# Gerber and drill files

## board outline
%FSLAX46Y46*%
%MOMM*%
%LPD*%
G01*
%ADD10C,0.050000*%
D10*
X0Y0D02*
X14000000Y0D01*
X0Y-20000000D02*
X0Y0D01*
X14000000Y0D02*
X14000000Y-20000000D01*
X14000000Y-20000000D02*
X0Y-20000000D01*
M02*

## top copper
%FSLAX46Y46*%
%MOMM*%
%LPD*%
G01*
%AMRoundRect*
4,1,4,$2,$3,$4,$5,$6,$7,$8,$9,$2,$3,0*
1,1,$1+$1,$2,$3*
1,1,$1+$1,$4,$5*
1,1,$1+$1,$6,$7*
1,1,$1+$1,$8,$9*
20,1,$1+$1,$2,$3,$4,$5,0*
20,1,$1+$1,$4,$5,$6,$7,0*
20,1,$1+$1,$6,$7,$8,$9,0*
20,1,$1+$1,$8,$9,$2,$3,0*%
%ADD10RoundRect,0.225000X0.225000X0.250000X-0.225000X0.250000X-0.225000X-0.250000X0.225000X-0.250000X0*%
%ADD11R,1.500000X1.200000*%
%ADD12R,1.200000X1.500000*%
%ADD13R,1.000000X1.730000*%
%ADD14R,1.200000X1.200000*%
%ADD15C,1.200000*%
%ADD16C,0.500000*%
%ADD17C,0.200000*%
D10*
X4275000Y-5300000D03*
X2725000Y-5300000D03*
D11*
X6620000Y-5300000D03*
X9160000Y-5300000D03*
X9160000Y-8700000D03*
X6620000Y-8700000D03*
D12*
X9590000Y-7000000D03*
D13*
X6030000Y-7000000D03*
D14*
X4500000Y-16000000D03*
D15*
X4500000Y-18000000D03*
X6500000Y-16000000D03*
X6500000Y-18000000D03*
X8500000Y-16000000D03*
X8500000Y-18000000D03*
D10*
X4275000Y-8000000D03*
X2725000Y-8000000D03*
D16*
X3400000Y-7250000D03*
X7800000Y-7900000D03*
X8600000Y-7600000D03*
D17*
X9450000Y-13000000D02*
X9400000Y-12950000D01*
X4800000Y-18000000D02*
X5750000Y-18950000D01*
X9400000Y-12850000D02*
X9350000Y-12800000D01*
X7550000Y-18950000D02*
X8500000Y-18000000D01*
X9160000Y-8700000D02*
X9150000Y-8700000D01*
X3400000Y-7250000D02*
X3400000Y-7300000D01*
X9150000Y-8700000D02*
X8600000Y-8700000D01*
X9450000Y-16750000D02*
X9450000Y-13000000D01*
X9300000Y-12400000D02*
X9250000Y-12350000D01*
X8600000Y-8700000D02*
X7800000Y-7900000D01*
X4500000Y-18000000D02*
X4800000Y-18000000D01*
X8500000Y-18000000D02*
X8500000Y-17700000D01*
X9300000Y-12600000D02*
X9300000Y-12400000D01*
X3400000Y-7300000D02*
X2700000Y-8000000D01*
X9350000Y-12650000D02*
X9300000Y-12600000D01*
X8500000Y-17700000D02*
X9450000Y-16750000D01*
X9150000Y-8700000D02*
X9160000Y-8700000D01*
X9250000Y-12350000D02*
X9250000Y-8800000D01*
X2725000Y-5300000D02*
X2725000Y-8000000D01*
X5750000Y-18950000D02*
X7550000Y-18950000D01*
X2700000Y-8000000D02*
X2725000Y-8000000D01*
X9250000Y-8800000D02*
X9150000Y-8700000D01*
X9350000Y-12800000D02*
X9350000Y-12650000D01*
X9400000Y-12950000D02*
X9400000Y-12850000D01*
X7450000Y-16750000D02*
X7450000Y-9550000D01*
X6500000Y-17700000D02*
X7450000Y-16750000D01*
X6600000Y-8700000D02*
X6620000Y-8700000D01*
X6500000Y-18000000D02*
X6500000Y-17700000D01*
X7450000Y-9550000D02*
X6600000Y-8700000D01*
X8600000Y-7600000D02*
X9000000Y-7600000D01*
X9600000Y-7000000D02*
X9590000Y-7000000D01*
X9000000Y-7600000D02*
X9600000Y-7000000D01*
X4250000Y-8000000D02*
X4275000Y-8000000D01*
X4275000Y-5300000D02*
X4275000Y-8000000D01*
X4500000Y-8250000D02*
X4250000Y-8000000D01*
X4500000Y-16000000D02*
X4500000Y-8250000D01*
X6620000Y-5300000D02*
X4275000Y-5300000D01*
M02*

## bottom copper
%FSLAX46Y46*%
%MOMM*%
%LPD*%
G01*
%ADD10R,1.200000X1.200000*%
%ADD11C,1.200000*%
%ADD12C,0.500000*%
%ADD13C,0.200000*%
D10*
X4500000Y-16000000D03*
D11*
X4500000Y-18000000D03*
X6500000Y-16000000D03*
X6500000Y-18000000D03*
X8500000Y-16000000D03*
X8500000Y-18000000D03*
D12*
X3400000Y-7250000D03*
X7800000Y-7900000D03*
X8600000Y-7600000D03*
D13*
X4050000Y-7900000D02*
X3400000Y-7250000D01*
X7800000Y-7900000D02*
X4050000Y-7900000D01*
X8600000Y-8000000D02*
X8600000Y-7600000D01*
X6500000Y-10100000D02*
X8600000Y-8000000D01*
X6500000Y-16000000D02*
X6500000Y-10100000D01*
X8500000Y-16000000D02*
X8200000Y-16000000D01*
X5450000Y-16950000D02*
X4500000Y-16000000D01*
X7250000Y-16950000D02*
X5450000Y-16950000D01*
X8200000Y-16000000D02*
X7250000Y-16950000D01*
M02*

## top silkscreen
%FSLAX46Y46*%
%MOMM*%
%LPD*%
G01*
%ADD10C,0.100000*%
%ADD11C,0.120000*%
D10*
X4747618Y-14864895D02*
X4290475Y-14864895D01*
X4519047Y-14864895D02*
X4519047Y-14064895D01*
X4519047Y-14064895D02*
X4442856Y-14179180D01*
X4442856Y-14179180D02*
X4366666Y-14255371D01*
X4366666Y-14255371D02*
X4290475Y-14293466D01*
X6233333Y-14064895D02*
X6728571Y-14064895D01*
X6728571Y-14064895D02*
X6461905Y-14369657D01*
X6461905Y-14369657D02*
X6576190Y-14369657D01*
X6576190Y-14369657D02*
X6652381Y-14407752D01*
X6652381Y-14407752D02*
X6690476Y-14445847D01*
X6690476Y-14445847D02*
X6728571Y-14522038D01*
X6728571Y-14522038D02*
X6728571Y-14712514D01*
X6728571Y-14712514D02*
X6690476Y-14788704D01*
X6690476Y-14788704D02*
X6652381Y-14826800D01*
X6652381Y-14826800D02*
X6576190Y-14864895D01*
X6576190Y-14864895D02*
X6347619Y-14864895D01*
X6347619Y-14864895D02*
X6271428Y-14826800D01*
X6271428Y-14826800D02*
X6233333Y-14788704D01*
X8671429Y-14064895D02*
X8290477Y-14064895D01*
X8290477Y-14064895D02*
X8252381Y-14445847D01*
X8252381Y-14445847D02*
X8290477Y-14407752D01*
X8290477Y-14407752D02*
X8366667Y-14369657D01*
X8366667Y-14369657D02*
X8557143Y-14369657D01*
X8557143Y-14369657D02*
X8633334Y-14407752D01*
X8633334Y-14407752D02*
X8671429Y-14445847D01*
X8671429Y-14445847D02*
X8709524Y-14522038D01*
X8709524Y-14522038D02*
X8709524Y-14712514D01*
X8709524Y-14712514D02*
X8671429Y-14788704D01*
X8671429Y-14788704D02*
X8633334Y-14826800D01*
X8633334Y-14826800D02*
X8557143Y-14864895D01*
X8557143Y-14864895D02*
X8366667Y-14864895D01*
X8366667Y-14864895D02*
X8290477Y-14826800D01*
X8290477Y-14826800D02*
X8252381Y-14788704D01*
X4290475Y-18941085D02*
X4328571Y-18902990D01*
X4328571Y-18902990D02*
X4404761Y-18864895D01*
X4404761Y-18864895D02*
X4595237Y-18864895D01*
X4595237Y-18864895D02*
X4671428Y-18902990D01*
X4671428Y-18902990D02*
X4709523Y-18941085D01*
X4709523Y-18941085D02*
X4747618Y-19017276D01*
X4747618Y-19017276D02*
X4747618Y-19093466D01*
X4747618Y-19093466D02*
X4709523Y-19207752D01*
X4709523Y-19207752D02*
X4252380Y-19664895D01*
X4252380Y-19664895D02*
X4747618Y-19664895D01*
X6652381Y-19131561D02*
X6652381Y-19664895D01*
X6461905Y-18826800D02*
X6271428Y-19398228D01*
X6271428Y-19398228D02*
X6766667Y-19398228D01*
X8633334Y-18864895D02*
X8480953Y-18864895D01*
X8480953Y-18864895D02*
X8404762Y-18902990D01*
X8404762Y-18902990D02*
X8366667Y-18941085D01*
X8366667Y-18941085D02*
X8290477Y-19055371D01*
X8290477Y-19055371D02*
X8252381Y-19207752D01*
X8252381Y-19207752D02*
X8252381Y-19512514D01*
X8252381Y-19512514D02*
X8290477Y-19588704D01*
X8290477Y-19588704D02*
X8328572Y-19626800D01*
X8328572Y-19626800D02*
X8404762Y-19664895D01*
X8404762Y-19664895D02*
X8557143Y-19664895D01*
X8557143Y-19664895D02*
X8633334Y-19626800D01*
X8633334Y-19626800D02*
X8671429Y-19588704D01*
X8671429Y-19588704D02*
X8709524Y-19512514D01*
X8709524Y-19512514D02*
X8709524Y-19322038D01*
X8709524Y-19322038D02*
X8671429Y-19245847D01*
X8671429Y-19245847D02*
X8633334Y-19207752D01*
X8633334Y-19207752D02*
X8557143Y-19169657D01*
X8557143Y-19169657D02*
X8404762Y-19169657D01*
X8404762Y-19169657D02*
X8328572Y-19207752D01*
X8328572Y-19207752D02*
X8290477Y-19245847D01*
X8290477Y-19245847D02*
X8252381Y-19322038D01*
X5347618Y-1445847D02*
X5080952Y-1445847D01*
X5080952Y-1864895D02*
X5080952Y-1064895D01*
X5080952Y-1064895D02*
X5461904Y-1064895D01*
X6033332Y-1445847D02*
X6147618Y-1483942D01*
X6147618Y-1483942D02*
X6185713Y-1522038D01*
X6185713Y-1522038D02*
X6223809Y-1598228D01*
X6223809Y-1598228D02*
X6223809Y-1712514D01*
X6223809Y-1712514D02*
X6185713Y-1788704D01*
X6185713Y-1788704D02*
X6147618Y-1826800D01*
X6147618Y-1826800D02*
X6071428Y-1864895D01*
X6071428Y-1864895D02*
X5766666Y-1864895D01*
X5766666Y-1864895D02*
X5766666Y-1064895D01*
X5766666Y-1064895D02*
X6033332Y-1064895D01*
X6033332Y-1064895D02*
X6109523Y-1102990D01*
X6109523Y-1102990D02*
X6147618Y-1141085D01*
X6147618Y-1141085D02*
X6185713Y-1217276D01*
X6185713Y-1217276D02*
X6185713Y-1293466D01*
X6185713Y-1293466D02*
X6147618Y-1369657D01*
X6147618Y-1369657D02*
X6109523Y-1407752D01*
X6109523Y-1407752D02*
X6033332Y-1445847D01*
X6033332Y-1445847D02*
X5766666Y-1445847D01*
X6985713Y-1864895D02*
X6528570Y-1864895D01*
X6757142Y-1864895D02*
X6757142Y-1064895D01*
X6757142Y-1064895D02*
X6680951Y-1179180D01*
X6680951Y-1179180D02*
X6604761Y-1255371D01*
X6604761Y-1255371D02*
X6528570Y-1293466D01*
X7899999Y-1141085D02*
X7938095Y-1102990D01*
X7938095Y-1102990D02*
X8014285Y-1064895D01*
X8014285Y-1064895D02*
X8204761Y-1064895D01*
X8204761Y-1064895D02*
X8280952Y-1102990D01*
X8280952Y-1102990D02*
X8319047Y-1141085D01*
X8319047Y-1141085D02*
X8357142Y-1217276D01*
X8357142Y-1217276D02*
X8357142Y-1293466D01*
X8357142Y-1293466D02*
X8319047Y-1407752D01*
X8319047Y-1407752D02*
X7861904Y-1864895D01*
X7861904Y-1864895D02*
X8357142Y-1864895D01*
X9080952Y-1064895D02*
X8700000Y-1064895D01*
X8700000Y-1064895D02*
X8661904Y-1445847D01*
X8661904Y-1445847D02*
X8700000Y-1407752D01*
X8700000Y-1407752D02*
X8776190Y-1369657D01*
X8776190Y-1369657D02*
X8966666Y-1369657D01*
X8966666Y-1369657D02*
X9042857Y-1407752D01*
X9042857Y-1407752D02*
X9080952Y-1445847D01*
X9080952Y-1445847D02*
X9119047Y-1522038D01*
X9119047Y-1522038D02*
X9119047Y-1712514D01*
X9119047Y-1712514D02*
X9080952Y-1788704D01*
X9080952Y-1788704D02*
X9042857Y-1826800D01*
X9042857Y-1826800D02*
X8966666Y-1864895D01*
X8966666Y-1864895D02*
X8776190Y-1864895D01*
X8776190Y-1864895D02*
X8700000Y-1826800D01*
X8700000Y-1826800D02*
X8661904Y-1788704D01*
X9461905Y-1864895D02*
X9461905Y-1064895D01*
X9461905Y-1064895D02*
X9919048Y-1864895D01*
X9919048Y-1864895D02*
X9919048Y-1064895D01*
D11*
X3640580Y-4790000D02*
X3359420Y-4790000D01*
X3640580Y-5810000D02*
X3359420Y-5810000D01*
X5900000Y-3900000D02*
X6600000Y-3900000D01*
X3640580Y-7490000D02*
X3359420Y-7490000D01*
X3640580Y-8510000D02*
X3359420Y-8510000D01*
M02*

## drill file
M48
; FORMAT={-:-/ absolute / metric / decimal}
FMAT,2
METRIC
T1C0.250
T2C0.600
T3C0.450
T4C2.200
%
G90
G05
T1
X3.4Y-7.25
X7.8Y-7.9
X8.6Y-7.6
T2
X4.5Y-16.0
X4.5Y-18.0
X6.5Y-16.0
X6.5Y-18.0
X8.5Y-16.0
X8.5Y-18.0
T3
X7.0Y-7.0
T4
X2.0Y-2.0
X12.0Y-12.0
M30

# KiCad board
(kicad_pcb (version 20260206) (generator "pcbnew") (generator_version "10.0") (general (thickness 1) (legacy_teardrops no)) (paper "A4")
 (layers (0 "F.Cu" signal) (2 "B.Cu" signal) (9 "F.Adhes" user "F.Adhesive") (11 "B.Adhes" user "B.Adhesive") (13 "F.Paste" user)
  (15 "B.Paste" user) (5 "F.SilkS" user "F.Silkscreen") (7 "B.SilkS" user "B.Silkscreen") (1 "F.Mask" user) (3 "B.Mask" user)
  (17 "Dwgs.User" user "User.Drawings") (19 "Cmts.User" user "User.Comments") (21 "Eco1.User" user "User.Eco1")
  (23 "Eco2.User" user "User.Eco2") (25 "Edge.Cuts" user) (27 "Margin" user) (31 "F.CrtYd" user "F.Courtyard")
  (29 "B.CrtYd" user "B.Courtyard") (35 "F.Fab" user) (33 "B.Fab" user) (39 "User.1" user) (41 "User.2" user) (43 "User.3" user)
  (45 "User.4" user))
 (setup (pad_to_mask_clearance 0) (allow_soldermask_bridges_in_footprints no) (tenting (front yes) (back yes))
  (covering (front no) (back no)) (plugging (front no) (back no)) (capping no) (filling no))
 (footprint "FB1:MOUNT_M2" (layer "F.Cu") (at 2 2)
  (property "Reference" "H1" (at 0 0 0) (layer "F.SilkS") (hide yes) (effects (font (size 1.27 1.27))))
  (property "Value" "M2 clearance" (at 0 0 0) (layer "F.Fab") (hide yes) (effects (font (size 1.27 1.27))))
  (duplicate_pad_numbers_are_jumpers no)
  (pad "" np_thru_hole circle (at 0 0) (size 2.2 2.2) (drill 2.2) (layers "*.Cu")))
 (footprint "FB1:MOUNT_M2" (layer "F.Cu") (at 12 12)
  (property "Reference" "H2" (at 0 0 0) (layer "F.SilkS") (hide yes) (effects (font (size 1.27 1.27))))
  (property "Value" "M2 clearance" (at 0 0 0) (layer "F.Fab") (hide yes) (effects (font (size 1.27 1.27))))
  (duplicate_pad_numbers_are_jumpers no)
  (pad "" np_thru_hole circle (at 0 0) (size 2.2 2.2) (drill 2.2) (layers "*.Cu")))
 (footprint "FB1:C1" (layer "F.Cu") (at 3.5 5.3 180)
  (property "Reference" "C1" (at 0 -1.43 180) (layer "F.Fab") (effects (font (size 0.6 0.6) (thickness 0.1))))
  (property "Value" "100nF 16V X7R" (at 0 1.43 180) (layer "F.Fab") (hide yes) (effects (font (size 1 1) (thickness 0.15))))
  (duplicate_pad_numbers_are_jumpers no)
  (fp_line (start -0.14058 0.51) (end 0.14058 0.51) (stroke (width 0.12) (type solid)) (layer "F.SilkS"))
  (fp_line (start -0.14058 -0.51) (end 0.14058 -0.51) (stroke (width 0.12) (type solid)) (layer "F.SilkS"))
  (pad "1" smd roundrect (at -0.775 0 180) (size 0.9 0.95) (layers "F.Cu" "F.Mask" "F.Paste") (roundrect_rratio 0.25) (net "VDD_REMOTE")
   (solder_mask_margin 0.025))
  (pad "2" smd roundrect (at 0.775 0 180) (size 0.9 0.95) (layers "F.Cu" "F.Mask" "F.Paste") (roundrect_rratio 0.25) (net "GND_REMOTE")
   (solder_mask_margin 0.025)))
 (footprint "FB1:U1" (layer "F.Cu") (at 7 7)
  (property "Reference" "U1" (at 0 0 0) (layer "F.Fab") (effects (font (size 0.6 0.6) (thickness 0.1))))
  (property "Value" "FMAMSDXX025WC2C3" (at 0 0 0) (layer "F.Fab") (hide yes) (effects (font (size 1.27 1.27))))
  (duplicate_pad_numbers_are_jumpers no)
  (fp_line (start -1.1 -3.1) (end -0.4 -3.1) (stroke (width 0.12) (type default)) (layer "F.SilkS"))
  (pad "" np_thru_hole circle (at 0 0) (size 0.45 0.45) (drill 0.45) (layers "*.Cu") (solder_mask_margin 0.025))
  (pad "1" smd rect (at -0.38 -1.7) (size 1.5 1.2) (layers "F.Cu" "F.Mask" "F.Paste") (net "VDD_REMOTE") (solder_mask_margin 0.025)
   (thermal_bridge_angle 45))
  (pad "2" smd rect (at 2.16 -1.7) (size 1.5 1.2) (layers "F.Cu" "F.Mask" "F.Paste") (solder_mask_margin 0.025) (thermal_bridge_angle 45))
  (pad "3" smd rect (at 2.16 1.7) (size 1.5 1.2) (layers "F.Cu" "F.Mask" "F.Paste") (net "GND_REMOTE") (solder_mask_margin 0.025)
   (thermal_bridge_angle 45))
  (pad "4" smd rect (at -0.38 1.7) (size 1.5 1.2) (layers "F.Cu" "F.Mask" "F.Paste") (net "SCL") (solder_mask_margin 0.025)
   (thermal_bridge_angle 45))
  (pad "5" smd rect (at 2.59 0) (size 1.2 1.5) (layers "F.Cu" "F.Mask" "F.Paste") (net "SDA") (solder_mask_margin 0.025)
   (thermal_bridge_angle 45))
  (pad "6" smd rect (at -0.97 0) (size 1 1.73) (layers "F.Cu" "F.Mask" "F.Paste") (solder_mask_margin 0.025) (thermal_bridge_angle 45)))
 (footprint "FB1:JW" (layer "F.Cu") (at 0 0)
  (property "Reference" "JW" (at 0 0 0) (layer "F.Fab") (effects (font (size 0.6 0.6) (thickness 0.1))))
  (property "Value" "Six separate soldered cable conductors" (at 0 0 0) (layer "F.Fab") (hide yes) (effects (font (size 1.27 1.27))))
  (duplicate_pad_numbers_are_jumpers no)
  (pad "1" thru_hole rect (at 4.5 16) (size 1.2 1.2) (drill 0.6) (layers "*.Cu") (remove_unused_layers no) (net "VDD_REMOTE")
   (solder_mask_margin 0.025) (thermal_bridge_angle 45))
  (pad "2" thru_hole circle (at 4.5 18) (size 1.2 1.2) (drill 0.6) (layers "*.Cu") (remove_unused_layers no) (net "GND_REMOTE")
   (solder_mask_margin 0.025))
  (pad "3" thru_hole circle (at 6.5 16) (size 1.2 1.2) (drill 0.6) (layers "*.Cu") (remove_unused_layers no) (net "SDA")
   (solder_mask_margin 0.025))
  (pad "4" thru_hole circle (at 6.5 18) (size 1.2 1.2) (drill 0.6) (layers "*.Cu") (remove_unused_layers no) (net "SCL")
   (solder_mask_margin 0.025))
  (pad "5" thru_hole circle (at 8.5 16) (size 1.2 1.2) (drill 0.6) (layers "*.Cu") (remove_unused_layers no) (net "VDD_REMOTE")
   (solder_mask_margin 0.025))
  (pad "6" thru_hole circle (at 8.5 18) (size 1.2 1.2) (drill 0.6) (layers "*.Cu") (remove_unused_layers no) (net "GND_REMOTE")
   (solder_mask_margin 0.025)))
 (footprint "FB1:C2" (layer "F.Cu") (at 3.5 8 180)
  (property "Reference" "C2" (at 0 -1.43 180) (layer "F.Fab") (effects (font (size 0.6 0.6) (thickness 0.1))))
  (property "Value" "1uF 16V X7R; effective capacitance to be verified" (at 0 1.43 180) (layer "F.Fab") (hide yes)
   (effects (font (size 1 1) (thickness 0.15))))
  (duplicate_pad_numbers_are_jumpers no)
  (fp_line (start -0.14058 0.51) (end 0.14058 0.51) (stroke (width 0.12) (type solid)) (layer "F.SilkS"))
  (fp_line (start -0.14058 -0.51) (end 0.14058 -0.51) (stroke (width 0.12) (type solid)) (layer "F.SilkS"))
  (pad "1" smd roundrect (at -0.775 0 180) (size 0.9 0.95) (layers "F.Cu" "F.Mask" "F.Paste") (roundrect_rratio 0.25) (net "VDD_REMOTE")
   (solder_mask_margin 0.025))
  (pad "2" smd roundrect (at 0.775 0 180) (size 0.9 0.95) (layers "F.Cu" "F.Mask" "F.Paste") (roundrect_rratio 0.25) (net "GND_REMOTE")
   (solder_mask_margin 0.025)))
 (gr_line (start 0 0) (end 14 0) (stroke (width 0.05) (type default)) (layer "Edge.Cuts"))
 (gr_line (start 0 20) (end 0 0) (stroke (width 0.05) (type default)) (layer "Edge.Cuts"))
 (gr_line (start 14 0) (end 14 20) (stroke (width 0.05) (type default)) (layer "Edge.Cuts"))
 (gr_line (start 14 20) (end 0 20) (stroke (width 0.05) (type default)) (layer "Edge.Cuts"))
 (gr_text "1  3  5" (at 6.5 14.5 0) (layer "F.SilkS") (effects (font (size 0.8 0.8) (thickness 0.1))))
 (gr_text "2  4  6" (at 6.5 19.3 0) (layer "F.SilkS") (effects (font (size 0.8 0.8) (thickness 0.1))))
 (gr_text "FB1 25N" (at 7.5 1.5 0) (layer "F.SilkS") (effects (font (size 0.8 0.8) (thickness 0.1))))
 (segment (start 9.45 13) (end 9.4 12.95) (width 0.2) (layer "F.Cu") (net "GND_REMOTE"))
 (segment (start 4.8 18) (end 5.75 18.95) (width 0.2) (layer "F.Cu") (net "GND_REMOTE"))
 (segment (start 9.4 12.85) (end 9.35 12.8) (width 0.2) (layer "F.Cu") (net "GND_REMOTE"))
 (segment (start 7.55 18.95) (end 8.5 18) (width 0.2) (layer "F.Cu") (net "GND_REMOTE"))
 (segment (start 9.16 8.7) (end 9.15 8.7) (width 0.2) (layer "F.Cu") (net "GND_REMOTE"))
 (segment (start 3.4 7.25) (end 3.4 7.3) (width 0.2) (layer "F.Cu") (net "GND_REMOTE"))
 (segment (start 9.15 8.7) (end 8.6 8.7) (width 0.2) (layer "F.Cu") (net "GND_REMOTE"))
 (segment (start 9.45 16.75) (end 9.45 13) (width 0.2) (layer "F.Cu") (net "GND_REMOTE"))
 (segment (start 9.3 12.4) (end 9.25 12.35) (width 0.2) (layer "F.Cu") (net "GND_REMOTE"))
 (segment (start 8.6 8.7) (end 7.8 7.9) (width 0.2) (layer "F.Cu") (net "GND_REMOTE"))
 (segment (start 4.5 18) (end 4.8 18) (width 0.2) (layer "F.Cu") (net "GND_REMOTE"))
 (segment (start 8.5 18) (end 8.5 17.7) (width 0.2) (layer "F.Cu") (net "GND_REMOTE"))
 (segment (start 9.3 12.6) (end 9.3 12.4) (width 0.2) (layer "F.Cu") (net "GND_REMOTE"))
 (segment (start 3.4 7.3) (end 2.7 8) (width 0.2) (layer "F.Cu") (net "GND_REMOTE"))
 (segment (start 9.35 12.65) (end 9.3 12.6) (width 0.2) (layer "F.Cu") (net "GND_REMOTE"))
 (segment (start 8.5 17.7) (end 9.45 16.75) (width 0.2) (layer "F.Cu") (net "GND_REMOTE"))
 (segment (start 9.15 8.7) (end 9.16 8.7) (width 0.2) (layer "F.Cu") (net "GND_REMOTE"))
 (segment (start 9.25 12.35) (end 9.25 8.8) (width 0.2) (layer "F.Cu") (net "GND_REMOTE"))
 (segment (start 2.725 5.3) (end 2.725 8) (width 0.2) (layer "F.Cu") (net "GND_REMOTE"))
 (segment (start 5.75 18.95) (end 7.55 18.95) (width 0.2) (layer "F.Cu") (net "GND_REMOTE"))
 (segment (start 2.7 8) (end 2.725 8) (width 0.2) (layer "F.Cu") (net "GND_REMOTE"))
 (segment (start 9.25 8.8) (end 9.15 8.7) (width 0.2) (layer "F.Cu") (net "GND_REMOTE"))
 (segment (start 9.35 12.8) (end 9.35 12.65) (width 0.2) (layer "F.Cu") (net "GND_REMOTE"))
 (segment (start 9.4 12.95) (end 9.4 12.85) (width 0.2) (layer "F.Cu") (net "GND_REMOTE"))
 (via (at 3.4 7.25) (size 0.5) (drill 0.25) (layers "F.Cu" "B.Cu") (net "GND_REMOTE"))
 (via (at 7.8 7.9) (size 0.5) (drill 0.25) (layers "F.Cu" "B.Cu") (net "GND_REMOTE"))
 (segment (start 4.05 7.9) (end 3.4 7.25) (width 0.2) (layer "B.Cu") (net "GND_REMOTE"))
 (segment (start 7.8 7.9) (end 4.05 7.9) (width 0.2) (layer "B.Cu") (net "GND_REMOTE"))
 (segment (start 7.45 16.75) (end 7.45 9.55) (width 0.2) (layer "F.Cu") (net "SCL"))
 (segment (start 6.5 17.7) (end 7.45 16.75) (width 0.2) (layer "F.Cu") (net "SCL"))
 (segment (start 6.6 8.7) (end 6.62 8.7) (width 0.2) (layer "F.Cu") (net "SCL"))
 (segment (start 6.5 18) (end 6.5 17.7) (width 0.2) (layer "F.Cu") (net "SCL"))
 (segment (start 7.45 9.55) (end 6.6 8.7) (width 0.2) (layer "F.Cu") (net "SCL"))
 (segment (start 8.6 7.6) (end 9 7.6) (width 0.2) (layer "F.Cu") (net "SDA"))
 (segment (start 9.6 7) (end 9.59 7) (width 0.2) (layer "F.Cu") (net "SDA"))
 (segment (start 9 7.6) (end 9.6 7) (width 0.2) (layer "F.Cu") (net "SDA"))
 (via (at 8.6 7.6) (size 0.5) (drill 0.25) (layers "F.Cu" "B.Cu") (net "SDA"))
 (segment (start 8.6 8) (end 8.6 7.6) (width 0.2) (layer "B.Cu") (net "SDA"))
 (segment (start 6.5 10.1) (end 8.6 8) (width 0.2) (layer "B.Cu") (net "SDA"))
 (segment (start 6.5 16) (end 6.5 10.1) (width 0.2) (layer "B.Cu") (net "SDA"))
 (segment (start 4.25 8) (end 4.275 8) (width 0.2) (layer "F.Cu") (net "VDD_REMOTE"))
 (segment (start 4.275 5.3) (end 4.275 8) (width 0.2) (layer "F.Cu") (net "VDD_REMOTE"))
 (segment (start 4.5 8.25) (end 4.25 8) (width 0.2) (layer "F.Cu") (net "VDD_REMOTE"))
 (segment (start 4.5 16) (end 4.5 8.25) (width 0.2) (layer "F.Cu") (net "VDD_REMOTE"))
 (segment (start 6.62 5.3) (end 4.275 5.3) (width 0.2) (layer "F.Cu") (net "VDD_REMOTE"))
 (segment (start 8.5 16) (end 8.2 16) (width 0.2) (layer "B.Cu") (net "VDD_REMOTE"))
 (segment (start 5.45 16.95) (end 4.5 16) (width 0.2) (layer "B.Cu") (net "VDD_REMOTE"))
 (segment (start 7.25 16.95) (end 5.45 16.95) (width 0.2) (layer "B.Cu") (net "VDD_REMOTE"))
 (segment (start 8.2 16) (end 7.25 16.95) (width 0.2) (layer "B.Cu") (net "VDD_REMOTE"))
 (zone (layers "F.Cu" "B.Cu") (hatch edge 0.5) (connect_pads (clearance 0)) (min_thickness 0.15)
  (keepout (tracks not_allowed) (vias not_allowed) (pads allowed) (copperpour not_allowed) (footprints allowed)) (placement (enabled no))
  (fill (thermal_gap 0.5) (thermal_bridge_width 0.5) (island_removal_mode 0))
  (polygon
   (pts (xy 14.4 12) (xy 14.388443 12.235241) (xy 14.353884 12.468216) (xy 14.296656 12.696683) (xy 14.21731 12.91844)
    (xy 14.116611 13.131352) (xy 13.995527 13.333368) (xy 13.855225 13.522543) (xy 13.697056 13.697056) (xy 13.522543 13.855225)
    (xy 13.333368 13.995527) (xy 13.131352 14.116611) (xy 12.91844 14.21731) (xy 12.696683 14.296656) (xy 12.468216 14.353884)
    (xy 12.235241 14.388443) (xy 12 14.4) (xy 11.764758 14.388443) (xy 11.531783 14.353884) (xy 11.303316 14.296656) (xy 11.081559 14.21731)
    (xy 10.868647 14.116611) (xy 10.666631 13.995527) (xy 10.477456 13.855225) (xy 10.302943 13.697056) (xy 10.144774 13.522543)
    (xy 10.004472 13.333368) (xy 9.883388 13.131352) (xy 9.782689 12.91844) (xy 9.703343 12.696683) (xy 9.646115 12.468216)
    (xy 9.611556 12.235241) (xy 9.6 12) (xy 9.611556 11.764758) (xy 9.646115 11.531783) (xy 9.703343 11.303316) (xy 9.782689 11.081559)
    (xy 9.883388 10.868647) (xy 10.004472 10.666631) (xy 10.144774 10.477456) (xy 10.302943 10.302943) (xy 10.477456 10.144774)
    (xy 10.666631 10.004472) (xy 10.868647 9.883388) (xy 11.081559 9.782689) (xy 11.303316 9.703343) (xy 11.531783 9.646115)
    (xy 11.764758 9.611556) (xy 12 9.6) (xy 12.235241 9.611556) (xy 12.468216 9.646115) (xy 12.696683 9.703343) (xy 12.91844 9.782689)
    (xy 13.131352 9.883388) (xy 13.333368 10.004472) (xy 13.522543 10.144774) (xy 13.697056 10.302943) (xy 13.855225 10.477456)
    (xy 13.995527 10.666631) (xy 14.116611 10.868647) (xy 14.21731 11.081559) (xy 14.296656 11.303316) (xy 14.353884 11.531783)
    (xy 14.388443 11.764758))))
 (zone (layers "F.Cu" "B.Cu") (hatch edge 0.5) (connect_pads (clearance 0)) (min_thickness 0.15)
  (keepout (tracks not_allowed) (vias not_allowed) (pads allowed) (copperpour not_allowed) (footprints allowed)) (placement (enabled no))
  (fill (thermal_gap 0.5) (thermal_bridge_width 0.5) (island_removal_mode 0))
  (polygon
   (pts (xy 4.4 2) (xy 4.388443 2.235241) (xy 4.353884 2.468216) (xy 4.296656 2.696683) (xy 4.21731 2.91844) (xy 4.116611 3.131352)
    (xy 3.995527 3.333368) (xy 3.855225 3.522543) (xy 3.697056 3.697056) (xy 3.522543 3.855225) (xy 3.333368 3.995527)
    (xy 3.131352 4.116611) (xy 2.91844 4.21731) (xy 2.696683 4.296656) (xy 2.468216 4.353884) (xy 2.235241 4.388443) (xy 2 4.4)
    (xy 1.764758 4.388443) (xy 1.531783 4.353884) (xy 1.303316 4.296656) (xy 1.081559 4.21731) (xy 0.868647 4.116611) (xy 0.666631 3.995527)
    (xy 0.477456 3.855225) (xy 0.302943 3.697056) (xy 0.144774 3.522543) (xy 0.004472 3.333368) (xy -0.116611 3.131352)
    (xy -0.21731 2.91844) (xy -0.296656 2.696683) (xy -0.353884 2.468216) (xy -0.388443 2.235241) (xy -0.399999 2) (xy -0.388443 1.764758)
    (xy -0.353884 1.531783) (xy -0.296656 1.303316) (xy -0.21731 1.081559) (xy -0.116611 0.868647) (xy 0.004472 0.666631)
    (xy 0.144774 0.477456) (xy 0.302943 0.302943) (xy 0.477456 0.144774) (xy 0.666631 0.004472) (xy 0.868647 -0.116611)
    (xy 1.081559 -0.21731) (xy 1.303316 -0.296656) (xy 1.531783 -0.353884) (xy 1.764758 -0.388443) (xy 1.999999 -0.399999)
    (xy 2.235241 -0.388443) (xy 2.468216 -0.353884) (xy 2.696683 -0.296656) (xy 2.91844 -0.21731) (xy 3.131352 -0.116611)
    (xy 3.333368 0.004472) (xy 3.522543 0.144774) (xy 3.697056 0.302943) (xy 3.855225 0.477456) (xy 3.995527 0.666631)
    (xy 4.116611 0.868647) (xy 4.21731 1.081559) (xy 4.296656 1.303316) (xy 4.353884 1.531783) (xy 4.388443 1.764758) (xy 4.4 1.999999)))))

